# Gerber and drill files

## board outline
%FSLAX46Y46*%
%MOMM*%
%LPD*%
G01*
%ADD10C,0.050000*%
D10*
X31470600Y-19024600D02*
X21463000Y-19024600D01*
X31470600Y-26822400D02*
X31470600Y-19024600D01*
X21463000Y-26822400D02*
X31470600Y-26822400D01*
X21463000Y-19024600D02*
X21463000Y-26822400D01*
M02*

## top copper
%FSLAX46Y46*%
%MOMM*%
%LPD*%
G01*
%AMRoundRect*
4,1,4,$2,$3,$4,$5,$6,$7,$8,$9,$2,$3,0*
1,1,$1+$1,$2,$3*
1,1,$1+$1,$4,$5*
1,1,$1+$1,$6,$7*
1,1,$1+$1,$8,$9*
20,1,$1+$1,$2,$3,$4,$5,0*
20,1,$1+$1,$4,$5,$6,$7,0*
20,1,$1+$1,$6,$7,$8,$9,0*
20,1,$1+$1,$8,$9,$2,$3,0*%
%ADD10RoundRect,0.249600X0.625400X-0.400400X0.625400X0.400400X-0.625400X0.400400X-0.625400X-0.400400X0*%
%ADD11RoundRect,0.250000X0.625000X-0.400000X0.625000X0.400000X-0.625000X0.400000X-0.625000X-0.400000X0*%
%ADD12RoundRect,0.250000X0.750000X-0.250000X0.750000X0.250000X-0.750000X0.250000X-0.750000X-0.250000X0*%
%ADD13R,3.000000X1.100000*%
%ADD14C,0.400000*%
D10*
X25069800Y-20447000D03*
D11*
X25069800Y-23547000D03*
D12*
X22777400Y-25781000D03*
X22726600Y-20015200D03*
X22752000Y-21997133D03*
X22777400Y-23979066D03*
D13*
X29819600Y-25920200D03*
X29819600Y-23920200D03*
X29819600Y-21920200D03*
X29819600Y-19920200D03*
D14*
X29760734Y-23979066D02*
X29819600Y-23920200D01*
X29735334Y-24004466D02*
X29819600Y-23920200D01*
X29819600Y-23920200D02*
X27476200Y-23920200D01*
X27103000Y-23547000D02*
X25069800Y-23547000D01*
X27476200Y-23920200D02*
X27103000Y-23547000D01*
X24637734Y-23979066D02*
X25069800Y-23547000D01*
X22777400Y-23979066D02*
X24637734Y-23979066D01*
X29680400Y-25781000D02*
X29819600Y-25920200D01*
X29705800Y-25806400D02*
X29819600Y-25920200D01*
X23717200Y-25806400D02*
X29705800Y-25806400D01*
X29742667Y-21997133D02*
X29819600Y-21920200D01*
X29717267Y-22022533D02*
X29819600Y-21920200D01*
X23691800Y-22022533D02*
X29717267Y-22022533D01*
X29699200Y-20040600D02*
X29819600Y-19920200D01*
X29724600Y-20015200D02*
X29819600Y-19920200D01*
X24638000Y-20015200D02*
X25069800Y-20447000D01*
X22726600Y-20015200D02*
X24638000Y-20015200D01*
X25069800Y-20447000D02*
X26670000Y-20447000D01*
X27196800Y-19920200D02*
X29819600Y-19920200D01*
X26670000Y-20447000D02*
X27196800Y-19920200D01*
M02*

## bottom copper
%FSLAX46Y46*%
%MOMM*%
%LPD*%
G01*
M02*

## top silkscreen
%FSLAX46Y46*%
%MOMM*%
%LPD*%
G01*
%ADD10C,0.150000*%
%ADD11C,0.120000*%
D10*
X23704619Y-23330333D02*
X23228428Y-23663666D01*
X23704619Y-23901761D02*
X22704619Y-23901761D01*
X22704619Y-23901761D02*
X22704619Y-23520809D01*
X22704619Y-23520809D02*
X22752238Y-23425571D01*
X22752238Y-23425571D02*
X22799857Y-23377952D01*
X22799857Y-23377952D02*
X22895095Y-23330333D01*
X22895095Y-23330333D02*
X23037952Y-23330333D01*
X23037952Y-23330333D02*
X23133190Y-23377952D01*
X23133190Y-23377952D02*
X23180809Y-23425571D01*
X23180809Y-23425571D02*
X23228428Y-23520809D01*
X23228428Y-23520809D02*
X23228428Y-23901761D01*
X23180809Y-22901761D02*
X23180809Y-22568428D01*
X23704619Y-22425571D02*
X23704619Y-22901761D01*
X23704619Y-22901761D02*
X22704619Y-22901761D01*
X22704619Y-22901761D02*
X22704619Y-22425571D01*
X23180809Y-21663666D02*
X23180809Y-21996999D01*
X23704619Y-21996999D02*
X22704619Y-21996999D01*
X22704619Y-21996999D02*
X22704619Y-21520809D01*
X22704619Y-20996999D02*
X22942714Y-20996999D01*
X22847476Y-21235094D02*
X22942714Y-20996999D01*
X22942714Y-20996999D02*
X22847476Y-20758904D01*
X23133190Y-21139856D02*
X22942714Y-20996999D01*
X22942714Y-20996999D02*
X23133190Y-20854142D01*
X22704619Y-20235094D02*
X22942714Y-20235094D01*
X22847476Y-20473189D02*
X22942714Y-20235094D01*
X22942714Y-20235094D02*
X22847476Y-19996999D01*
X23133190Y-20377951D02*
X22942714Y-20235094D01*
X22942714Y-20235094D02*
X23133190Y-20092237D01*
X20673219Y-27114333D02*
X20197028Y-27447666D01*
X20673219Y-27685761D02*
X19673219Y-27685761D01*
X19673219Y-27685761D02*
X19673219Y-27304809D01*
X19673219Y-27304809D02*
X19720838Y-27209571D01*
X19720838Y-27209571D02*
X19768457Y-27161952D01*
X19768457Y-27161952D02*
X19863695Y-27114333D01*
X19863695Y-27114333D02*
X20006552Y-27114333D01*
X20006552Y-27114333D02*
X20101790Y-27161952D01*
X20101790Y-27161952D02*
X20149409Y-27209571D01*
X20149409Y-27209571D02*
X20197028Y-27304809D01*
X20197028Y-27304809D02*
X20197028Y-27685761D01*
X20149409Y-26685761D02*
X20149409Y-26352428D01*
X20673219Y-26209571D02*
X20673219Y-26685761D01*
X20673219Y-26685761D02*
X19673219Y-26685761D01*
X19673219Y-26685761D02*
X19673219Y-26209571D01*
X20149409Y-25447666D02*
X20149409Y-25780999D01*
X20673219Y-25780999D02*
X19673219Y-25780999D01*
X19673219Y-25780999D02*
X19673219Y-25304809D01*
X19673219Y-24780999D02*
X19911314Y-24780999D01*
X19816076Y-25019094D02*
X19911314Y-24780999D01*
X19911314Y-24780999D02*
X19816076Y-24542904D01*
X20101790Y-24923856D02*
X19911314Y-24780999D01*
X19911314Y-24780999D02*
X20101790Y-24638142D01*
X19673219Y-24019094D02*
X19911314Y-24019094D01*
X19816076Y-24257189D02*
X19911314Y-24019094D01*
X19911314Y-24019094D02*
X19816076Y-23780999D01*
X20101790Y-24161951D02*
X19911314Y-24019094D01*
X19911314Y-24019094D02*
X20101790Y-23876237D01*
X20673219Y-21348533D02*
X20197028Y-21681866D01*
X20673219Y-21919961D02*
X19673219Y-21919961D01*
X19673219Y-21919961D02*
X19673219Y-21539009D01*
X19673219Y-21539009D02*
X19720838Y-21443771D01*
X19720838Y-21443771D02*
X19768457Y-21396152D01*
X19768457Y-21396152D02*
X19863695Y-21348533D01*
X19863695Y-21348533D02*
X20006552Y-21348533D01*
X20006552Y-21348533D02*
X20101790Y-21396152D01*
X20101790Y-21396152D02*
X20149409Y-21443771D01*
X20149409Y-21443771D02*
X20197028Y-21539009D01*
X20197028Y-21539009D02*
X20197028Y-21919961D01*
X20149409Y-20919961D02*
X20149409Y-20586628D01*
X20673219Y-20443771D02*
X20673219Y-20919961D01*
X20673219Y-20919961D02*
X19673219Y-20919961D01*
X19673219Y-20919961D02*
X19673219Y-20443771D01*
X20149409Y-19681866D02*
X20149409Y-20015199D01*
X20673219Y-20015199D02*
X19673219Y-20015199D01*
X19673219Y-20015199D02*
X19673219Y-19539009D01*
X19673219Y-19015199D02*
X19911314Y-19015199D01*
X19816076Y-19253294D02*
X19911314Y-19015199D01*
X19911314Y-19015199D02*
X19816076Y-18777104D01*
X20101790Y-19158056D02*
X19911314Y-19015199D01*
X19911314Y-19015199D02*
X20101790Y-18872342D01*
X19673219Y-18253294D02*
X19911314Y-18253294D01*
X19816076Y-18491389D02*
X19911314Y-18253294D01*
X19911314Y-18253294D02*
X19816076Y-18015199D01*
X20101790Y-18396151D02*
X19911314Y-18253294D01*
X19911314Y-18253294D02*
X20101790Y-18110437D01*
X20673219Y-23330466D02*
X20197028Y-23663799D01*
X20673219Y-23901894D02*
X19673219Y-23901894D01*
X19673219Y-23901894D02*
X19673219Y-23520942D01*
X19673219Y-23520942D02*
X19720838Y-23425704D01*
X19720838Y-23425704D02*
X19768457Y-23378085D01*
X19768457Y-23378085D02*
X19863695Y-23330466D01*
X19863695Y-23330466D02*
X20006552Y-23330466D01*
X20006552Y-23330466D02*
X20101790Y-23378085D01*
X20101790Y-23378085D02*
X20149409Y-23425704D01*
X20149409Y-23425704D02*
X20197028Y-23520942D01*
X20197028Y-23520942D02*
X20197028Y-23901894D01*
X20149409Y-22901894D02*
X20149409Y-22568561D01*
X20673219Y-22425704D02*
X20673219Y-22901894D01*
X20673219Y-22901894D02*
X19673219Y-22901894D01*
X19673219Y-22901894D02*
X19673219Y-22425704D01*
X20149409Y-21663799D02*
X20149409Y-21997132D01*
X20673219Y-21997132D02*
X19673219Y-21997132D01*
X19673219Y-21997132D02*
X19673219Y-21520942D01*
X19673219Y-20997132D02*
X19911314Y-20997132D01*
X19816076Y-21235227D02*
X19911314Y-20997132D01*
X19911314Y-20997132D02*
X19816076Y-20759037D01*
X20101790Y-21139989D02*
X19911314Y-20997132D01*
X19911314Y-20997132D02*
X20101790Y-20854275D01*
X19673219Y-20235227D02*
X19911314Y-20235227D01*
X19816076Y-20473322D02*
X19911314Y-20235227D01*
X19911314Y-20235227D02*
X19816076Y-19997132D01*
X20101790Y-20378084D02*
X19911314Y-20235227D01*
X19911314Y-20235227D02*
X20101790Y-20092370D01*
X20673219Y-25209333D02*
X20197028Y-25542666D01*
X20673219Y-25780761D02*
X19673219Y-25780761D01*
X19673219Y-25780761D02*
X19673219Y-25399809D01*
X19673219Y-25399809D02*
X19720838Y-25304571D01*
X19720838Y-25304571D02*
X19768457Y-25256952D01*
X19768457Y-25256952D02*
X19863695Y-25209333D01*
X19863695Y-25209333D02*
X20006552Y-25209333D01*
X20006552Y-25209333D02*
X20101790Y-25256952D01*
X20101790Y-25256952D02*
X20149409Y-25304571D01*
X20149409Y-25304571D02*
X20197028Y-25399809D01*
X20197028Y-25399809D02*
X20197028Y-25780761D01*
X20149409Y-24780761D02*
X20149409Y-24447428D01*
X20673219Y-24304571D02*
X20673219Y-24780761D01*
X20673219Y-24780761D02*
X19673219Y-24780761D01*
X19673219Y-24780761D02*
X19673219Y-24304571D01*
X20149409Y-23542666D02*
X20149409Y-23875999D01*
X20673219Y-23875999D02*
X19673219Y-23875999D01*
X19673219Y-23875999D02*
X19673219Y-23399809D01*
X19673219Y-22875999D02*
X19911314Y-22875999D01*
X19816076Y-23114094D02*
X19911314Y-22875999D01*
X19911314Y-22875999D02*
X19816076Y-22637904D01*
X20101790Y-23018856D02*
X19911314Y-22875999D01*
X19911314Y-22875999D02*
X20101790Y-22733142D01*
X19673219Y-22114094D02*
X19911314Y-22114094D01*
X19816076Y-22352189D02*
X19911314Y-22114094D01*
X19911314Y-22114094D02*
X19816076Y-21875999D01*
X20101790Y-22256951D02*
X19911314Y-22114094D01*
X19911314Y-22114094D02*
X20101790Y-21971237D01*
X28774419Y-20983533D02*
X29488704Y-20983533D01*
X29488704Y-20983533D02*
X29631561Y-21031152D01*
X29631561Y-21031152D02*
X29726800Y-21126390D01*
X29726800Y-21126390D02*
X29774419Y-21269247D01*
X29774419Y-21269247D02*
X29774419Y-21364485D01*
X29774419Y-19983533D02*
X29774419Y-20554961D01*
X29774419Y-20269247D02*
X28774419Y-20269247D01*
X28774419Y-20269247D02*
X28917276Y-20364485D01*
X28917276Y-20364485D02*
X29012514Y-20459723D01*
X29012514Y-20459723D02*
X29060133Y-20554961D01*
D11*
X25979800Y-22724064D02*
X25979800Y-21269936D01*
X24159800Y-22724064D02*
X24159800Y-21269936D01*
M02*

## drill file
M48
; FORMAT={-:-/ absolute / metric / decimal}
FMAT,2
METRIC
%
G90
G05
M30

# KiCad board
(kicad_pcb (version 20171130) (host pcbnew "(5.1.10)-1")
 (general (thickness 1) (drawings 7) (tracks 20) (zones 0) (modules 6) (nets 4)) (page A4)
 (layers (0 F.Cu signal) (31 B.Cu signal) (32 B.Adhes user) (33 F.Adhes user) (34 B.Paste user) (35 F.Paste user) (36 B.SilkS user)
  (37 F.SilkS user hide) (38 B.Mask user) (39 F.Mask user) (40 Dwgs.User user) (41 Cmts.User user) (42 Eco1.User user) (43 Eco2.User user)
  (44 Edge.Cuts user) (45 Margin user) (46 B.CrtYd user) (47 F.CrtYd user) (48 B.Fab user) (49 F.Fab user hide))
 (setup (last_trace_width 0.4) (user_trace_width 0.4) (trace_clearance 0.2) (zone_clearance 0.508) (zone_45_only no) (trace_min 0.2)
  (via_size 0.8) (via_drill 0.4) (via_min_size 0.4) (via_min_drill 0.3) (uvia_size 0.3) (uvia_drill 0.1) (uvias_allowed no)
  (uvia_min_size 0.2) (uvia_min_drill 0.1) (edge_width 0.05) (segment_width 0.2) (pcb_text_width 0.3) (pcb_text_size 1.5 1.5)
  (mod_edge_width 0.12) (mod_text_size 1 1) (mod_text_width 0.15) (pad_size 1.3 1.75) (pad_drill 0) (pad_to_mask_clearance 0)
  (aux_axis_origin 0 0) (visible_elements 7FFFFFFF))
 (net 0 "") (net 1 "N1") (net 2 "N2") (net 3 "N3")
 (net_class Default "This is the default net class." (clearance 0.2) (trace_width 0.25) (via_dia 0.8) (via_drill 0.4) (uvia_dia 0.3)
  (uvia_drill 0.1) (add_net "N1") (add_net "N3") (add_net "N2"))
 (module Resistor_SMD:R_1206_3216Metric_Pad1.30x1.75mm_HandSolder (layer F.Cu) (at 25.0698 21.997 90)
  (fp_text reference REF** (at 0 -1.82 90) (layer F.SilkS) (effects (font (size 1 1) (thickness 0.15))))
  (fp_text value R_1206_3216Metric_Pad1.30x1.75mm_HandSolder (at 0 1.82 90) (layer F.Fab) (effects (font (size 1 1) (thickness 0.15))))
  (fp_line (start -0.727064 0.91) (end 0.727064 0.91) (layer F.SilkS) (width 0.12))
  (fp_line (start -0.727064 -0.91) (end 0.727064 -0.91) (layer F.SilkS) (width 0.12))
  (pad 2 smd roundrect (at 1.55 0 90) (size 1.3 1.75) (layers F.Cu F.Paste F.Mask) (roundrect_rratio 0.192) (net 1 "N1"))
  (pad 1 smd roundrect (at -1.55 0 90) (size 1.3 1.75) (layers F.Cu F.Paste F.Mask) (roundrect_rratio 0.1923076923076923)))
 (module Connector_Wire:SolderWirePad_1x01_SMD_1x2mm (layer F.Cu) (at 22.7584 25.781 90)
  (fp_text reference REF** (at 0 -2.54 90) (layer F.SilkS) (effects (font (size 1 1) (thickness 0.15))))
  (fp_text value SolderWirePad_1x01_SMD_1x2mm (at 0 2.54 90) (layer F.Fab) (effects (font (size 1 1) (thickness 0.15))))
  (pad 4 smd roundrect (at 0 0.019 90) (size 1 2) (layers F.Cu F.Paste F.Mask) (roundrect_rratio 0.25) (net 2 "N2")))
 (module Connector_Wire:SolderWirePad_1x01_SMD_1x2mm (layer F.Cu) (at 22.7584 20.0152 90)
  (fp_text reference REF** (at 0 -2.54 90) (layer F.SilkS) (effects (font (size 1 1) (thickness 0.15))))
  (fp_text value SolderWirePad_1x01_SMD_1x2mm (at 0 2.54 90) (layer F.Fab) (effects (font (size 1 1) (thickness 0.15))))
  (pad 1 smd roundrect (at 0 -0.0318 90) (size 1 2) (layers F.Cu F.Paste F.Mask) (roundrect_rratio 0.25) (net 1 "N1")))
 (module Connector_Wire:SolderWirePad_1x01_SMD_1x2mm (layer F.Cu) (at 22.7584 21.997133 90)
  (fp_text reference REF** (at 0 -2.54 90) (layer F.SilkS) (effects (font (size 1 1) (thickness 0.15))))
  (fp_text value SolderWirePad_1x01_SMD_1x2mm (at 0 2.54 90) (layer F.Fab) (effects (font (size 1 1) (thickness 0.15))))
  (pad 2 smd roundrect (at 0 -0.0064 90) (size 1 2) (layers F.Cu F.Paste F.Mask) (roundrect_rratio 0.25) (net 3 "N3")))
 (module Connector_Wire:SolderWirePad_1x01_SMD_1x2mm (layer F.Cu) (at 22.7584 23.876 90)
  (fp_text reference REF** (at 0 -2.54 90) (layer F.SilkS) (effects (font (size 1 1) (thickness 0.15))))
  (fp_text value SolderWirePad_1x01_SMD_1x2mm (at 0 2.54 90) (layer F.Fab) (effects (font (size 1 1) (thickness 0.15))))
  (pad 4 smd roundrect (at -0.103066 0.019 90) (size 1 2) (layers F.Cu F.Paste F.Mask) (roundrect_rratio 0.25)))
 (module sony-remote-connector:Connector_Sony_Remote (layer F.Cu) (at 28.5496 21.9202 270)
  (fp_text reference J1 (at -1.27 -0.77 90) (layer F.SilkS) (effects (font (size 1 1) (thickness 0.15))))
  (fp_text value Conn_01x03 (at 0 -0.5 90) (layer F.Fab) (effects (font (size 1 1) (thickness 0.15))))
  (pad 4 smd rect (at 4 -1.27 270) (size 1.1 3) (layers F.Cu F.Paste F.Mask) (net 2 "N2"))
  (pad 3 smd rect (at 2 -1.27 270) (size 1.1 3) (layers F.Cu F.Paste F.Mask))
  (pad 2 smd rect (at 0 -1.27 270) (size 1.1 3) (layers F.Cu F.Paste F.Mask) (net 3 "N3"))
  (pad 1 smd rect (at -2 -1.27 270) (size 1.1 3) (layers F.Cu F.Paste F.Mask) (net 1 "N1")))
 (gr_line (start 31.4706 19.0246) (end 21.463 19.0246) (layer Edge.Cuts) (width 0.05))
 (gr_line (start 31.4706 26.8224) (end 31.4706 19.0246) (layer Edge.Cuts) (width 0.05))
 (gr_line (start 21.463 26.8224) (end 31.4706 26.8224) (layer Edge.Cuts) (width 0.05))
 (gr_line (start 21.463 19.0246) (end 21.463 26.8224) (layer Edge.Cuts) (width 0.05))
 (segment (start 29.760734 23.979066) (end 29.8196 23.9202) (width 0.4) (layer F.Cu) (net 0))
 (segment (start 29.735334 24.004466) (end 29.8196 23.9202) (width 0.4) (layer F.Cu) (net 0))
 (segment (start 29.8196 23.9202) (end 27.4762 23.9202) (width 0.4) (layer F.Cu) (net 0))
 (segment (start 27.103 23.547) (end 25.0698 23.547) (width 0.4) (layer F.Cu) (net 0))
 (segment (start 27.4762 23.9202) (end 27.103 23.547) (width 0.4) (layer F.Cu) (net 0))
 (segment (start 24.637734 23.979066) (end 25.0698 23.547) (width 0.4) (layer F.Cu) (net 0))
 (segment (start 22.7774 23.979066) (end 24.637734 23.979066) (width 0.4) (layer F.Cu) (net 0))
 (segment (start 29.6804 25.781) (end 29.8196 25.9202) (width 0.4) (layer F.Cu) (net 2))
 (segment (start 29.7058 25.8064) (end 29.8196 25.9202) (width 0.4) (layer F.Cu) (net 2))
 (segment (start 23.7172 25.8064) (end 29.7058 25.8064) (width 0.4) (layer F.Cu) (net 2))
 (segment (start 29.742667 21.997133) (end 29.8196 21.9202) (width 0.4) (layer F.Cu) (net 3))
 (segment (start 29.717267 22.022533) (end 29.8196 21.9202) (width 0.4) (layer F.Cu) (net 3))
 (segment (start 23.6918 22.022533) (end 29.717267 22.022533) (width 0.4) (layer F.Cu) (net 3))
 (segment (start 29.6992 20.0406) (end 29.8196 19.9202) (width 0.4) (layer F.Cu) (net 1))
 (segment (start 29.7246 20.0152) (end 29.8196 19.9202) (width 0.4) (layer F.Cu) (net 1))
 (segment (start 24.638 20.0152) (end 25.0698 20.447) (width 0.4) (layer F.Cu) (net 1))
 (segment (start 22.7266 20.0152) (end 24.638 20.0152) (width 0.4) (layer F.Cu) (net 1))
 (segment (start 25.0698 20.447) (end 26.67 20.447) (width 0.4) (layer F.Cu) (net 1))
 (segment (start 27.1968 19.9202) (end 29.8196 19.9202) (width 0.4) (layer F.Cu) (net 1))
 (segment (start 26.67 20.447) (end 27.1968 19.9202) (width 0.4) (layer F.Cu) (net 1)))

